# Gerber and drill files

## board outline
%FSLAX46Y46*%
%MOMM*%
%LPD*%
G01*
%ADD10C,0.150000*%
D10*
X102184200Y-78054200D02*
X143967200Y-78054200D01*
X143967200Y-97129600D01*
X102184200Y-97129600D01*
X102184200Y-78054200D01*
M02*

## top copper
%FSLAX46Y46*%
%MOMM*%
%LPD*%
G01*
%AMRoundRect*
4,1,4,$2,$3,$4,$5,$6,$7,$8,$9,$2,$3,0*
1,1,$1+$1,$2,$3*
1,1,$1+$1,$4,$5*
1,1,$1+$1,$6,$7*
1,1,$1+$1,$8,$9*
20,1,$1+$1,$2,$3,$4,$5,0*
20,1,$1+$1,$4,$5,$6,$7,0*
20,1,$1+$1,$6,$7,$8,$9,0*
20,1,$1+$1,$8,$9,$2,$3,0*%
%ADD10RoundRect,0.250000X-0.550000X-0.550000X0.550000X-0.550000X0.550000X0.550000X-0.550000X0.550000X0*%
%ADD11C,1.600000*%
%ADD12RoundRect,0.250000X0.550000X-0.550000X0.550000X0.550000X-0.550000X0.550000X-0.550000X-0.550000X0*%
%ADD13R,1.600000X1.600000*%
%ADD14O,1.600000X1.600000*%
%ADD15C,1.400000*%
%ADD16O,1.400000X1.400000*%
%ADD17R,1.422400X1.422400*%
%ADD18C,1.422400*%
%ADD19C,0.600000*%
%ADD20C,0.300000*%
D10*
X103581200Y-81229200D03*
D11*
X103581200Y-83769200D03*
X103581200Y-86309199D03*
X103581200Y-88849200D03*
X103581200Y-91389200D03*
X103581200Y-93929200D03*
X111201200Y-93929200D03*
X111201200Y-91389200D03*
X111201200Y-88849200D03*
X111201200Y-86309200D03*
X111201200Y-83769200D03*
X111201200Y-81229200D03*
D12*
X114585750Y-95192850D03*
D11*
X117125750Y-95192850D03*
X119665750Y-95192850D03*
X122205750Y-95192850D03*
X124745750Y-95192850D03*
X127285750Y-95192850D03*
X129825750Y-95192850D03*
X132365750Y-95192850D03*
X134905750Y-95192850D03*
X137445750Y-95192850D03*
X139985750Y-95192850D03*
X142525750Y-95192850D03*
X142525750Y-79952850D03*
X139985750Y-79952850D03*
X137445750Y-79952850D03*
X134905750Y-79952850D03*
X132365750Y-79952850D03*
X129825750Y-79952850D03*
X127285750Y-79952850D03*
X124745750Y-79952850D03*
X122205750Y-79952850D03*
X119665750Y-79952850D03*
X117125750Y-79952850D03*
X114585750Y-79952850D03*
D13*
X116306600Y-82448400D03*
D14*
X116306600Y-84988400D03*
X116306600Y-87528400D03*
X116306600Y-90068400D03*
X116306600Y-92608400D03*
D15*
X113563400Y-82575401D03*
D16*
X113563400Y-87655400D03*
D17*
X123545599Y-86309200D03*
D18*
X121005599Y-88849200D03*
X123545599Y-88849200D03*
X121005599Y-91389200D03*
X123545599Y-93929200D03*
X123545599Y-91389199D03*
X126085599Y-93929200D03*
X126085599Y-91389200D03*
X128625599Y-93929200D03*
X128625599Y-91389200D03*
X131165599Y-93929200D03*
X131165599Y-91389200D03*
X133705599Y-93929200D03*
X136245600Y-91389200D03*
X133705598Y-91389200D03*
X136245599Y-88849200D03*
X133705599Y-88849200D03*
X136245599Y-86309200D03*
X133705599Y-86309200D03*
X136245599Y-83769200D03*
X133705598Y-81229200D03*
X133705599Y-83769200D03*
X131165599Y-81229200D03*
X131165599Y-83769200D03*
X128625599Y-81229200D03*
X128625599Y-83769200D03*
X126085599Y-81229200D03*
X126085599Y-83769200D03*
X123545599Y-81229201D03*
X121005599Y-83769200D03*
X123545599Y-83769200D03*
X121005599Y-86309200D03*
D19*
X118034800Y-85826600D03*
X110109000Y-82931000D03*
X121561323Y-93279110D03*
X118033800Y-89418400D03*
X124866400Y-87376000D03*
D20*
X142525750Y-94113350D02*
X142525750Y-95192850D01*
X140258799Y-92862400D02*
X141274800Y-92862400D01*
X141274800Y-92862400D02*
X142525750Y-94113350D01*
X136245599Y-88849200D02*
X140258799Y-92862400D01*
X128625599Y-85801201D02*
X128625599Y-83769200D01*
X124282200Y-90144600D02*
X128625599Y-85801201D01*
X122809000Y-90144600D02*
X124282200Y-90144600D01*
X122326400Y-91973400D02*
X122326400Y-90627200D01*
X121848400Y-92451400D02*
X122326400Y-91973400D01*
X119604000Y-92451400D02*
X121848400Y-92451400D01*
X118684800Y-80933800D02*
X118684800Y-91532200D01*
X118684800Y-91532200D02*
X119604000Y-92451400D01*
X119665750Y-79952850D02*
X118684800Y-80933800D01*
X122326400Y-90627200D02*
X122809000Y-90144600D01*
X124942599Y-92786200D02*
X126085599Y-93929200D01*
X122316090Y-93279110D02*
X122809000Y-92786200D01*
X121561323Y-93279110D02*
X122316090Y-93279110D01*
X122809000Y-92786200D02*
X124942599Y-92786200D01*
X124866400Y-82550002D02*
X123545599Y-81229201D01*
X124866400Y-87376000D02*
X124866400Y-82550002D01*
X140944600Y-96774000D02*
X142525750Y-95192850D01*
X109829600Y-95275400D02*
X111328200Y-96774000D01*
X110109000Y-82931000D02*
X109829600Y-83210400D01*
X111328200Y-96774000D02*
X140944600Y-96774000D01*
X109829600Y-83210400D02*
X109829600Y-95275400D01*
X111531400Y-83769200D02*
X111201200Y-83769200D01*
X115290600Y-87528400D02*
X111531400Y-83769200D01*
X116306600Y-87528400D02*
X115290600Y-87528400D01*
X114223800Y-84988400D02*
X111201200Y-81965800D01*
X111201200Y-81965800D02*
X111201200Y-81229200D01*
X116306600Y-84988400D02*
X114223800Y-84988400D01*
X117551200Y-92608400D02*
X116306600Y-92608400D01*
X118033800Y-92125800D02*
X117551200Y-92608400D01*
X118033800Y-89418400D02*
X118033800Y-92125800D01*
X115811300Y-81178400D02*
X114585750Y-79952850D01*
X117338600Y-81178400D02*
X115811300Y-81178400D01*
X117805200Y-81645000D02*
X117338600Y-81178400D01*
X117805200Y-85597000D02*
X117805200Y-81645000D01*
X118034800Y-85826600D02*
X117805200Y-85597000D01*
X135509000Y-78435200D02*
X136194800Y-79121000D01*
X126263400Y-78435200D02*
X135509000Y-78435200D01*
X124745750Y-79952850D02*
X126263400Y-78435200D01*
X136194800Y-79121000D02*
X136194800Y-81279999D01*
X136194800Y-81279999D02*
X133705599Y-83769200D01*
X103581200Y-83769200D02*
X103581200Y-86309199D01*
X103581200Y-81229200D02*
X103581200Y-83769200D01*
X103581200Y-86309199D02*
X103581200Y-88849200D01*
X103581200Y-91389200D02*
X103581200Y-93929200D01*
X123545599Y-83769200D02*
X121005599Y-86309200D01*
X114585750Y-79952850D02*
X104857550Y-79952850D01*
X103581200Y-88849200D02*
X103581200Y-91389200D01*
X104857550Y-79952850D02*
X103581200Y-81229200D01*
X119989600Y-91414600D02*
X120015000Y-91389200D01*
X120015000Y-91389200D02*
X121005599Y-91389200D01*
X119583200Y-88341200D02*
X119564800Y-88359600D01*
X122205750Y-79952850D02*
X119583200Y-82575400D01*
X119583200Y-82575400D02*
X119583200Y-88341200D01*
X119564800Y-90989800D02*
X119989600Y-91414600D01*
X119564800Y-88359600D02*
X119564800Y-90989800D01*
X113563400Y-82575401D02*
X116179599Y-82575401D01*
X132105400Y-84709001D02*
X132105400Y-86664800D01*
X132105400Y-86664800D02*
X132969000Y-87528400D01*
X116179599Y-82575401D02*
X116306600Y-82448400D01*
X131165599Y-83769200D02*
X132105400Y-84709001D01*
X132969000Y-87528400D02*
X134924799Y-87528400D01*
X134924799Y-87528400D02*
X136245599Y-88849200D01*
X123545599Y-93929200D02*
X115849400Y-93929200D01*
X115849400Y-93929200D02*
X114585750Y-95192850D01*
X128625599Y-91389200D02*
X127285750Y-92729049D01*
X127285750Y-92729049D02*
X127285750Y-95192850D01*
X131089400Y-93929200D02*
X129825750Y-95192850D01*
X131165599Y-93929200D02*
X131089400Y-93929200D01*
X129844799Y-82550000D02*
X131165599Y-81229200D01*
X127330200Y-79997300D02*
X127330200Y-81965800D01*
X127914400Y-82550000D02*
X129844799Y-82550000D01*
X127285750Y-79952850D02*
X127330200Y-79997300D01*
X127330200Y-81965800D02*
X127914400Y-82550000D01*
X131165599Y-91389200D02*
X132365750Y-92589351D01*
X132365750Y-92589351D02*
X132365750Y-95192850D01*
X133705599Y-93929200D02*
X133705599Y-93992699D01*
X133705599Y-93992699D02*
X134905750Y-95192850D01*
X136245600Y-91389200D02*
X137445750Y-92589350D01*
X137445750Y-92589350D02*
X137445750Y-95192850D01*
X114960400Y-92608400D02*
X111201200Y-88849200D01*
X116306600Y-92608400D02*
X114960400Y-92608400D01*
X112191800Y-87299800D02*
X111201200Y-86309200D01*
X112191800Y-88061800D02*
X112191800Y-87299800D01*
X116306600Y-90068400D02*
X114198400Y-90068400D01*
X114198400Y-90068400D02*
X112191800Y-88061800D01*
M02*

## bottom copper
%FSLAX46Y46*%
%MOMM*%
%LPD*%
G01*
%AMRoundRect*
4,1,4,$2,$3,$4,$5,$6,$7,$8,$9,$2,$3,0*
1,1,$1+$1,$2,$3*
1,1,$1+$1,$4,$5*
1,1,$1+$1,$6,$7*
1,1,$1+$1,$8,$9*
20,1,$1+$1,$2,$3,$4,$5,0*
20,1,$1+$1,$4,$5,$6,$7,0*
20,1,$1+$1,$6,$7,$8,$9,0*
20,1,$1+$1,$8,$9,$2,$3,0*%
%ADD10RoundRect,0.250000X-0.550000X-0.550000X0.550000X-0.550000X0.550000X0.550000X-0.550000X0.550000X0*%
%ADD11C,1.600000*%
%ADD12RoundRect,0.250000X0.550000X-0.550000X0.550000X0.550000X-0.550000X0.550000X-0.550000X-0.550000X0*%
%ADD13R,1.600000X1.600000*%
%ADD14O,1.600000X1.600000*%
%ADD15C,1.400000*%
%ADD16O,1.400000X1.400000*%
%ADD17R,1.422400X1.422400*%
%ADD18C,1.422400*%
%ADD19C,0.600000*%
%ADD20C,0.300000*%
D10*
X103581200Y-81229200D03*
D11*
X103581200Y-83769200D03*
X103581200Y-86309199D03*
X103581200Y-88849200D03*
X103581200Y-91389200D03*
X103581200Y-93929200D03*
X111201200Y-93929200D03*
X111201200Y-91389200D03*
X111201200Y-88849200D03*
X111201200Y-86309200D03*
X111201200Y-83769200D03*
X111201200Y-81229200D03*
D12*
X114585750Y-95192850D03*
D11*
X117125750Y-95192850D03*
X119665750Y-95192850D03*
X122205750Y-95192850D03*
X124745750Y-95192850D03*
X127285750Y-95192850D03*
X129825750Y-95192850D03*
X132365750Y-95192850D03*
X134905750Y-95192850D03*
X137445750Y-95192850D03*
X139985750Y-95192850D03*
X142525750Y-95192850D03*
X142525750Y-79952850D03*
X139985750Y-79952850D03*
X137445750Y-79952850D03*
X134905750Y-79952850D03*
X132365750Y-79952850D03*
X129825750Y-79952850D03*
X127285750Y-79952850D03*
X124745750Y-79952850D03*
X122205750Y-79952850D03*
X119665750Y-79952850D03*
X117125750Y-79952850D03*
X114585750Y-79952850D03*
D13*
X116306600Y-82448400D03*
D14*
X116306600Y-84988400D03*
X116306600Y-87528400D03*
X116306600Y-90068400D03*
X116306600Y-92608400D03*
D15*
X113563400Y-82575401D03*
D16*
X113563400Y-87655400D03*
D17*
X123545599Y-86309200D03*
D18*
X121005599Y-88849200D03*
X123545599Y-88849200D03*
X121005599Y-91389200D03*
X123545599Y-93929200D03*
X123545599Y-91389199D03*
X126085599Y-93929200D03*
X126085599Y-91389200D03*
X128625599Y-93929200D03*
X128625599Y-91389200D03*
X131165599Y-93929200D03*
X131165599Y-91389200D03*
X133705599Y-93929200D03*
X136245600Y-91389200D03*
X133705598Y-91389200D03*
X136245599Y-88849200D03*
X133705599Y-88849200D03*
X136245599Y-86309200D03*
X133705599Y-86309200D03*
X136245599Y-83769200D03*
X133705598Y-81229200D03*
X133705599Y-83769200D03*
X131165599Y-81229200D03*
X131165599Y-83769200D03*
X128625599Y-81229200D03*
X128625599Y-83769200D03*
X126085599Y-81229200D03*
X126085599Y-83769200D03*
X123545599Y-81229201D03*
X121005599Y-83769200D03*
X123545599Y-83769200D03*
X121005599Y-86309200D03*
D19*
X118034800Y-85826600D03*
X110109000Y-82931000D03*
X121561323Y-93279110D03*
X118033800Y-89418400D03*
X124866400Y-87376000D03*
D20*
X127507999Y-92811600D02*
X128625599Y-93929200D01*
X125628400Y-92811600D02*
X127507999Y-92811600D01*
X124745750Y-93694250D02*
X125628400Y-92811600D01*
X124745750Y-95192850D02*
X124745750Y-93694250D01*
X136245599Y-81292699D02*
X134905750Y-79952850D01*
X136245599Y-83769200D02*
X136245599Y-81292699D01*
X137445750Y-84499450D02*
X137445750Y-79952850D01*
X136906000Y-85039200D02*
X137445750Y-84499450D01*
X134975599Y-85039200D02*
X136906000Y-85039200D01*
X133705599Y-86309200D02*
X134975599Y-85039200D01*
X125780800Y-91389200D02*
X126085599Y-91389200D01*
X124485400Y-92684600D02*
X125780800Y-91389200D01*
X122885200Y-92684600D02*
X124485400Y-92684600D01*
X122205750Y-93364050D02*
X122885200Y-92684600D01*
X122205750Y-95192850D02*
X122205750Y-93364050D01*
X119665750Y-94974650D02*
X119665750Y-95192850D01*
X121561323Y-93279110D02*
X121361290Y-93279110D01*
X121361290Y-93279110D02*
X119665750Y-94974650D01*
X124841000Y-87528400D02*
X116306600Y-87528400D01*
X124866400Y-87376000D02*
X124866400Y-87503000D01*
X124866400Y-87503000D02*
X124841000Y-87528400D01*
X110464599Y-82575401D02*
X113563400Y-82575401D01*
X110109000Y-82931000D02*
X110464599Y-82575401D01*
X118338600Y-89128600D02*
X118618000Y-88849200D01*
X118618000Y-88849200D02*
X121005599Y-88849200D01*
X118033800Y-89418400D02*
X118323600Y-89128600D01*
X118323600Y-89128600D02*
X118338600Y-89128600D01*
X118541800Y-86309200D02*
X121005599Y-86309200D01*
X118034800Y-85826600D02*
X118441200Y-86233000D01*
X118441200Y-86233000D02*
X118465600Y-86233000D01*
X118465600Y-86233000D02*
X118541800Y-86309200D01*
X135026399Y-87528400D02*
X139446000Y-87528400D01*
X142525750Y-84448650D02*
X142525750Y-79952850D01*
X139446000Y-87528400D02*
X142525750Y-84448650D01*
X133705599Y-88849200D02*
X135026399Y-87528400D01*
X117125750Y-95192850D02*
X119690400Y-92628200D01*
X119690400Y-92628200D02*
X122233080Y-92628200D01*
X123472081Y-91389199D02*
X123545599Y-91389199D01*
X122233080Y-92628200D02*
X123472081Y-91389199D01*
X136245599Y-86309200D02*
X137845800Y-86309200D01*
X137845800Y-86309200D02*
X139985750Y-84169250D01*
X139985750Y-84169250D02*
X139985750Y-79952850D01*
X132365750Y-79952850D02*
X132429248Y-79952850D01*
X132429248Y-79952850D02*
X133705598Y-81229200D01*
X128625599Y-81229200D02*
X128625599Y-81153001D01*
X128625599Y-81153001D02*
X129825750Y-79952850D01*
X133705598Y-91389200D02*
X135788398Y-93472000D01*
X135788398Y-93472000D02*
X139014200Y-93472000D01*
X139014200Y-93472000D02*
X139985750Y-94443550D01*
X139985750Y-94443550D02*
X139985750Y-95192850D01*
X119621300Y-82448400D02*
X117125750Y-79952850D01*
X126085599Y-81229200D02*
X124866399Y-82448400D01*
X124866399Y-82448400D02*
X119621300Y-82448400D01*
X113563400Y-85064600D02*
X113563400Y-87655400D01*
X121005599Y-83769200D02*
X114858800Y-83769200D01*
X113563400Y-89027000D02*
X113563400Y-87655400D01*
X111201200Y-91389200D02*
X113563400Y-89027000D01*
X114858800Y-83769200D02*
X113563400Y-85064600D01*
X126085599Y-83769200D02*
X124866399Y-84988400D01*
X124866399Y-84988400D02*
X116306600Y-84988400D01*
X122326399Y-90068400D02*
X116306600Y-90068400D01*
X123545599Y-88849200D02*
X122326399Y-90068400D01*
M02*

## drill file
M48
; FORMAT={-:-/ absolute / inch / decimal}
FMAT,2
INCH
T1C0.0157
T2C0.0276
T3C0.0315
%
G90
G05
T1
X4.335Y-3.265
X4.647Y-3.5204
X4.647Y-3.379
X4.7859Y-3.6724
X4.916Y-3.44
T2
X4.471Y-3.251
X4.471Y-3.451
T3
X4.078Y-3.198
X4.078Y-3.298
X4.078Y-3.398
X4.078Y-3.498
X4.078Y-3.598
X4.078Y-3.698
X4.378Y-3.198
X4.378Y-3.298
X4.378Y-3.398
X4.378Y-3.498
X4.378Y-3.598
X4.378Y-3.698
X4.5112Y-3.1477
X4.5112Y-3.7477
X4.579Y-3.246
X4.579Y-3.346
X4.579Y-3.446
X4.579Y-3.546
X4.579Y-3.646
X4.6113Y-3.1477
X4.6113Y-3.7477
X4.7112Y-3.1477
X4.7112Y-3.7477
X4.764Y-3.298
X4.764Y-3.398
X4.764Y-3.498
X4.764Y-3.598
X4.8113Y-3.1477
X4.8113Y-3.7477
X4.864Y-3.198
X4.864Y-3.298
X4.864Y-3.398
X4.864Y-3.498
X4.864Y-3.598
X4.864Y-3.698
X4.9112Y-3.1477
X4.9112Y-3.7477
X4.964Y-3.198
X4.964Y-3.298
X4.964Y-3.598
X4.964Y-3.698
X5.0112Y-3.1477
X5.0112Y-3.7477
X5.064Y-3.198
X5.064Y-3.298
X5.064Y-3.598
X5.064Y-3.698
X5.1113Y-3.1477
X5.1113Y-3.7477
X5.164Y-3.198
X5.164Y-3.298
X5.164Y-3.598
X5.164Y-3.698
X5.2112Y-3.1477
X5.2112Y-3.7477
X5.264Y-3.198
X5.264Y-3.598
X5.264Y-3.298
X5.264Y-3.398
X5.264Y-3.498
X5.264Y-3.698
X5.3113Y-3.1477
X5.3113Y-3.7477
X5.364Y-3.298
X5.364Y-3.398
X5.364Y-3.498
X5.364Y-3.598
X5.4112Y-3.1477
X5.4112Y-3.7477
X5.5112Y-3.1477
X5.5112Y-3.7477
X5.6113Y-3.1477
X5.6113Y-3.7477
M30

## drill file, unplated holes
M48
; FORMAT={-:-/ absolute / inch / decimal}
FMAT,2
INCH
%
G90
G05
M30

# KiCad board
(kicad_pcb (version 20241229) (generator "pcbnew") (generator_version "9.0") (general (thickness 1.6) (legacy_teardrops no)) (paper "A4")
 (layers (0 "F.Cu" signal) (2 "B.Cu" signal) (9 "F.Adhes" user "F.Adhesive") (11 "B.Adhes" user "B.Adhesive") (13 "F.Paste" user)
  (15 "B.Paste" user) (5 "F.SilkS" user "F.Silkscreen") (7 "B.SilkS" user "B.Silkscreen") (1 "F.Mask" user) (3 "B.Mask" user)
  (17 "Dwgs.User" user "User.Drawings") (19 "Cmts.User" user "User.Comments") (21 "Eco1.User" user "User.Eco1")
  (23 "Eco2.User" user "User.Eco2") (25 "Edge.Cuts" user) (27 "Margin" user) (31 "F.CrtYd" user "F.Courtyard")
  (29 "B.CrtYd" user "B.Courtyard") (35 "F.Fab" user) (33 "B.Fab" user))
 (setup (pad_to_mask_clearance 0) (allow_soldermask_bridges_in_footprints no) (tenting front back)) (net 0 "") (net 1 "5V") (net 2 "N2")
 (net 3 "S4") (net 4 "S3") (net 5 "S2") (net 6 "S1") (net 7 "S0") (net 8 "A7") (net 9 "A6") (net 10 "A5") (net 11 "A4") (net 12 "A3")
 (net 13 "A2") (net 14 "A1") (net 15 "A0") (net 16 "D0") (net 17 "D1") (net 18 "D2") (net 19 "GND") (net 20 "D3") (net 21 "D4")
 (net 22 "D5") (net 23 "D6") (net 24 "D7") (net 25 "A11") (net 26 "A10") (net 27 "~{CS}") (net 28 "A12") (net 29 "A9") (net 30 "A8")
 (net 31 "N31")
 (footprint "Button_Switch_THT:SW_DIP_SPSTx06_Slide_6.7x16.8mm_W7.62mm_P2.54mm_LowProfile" (layer "F.Cu") (at 103.5812 81.2292)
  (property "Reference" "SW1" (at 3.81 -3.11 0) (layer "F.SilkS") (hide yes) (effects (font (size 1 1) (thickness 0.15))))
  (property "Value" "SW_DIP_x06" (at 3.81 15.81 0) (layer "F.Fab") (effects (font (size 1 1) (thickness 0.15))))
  (pad "1" thru_hole roundrect (at 0 0) (size 1.6 1.6) (drill 0.8) (layers "*.Cu" "*.Mask") (remove_unused_layers no)
   (roundrect_rratio 0.15625) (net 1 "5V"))
  (pad "2" thru_hole circle (at 0 2.54) (size 1.6 1.6) (drill 0.8) (layers "*.Cu" "*.Mask") (remove_unused_layers no) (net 1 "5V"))
  (pad "3" thru_hole circle (at 0 5.079999) (size 1.6 1.6) (drill 0.8) (layers "*.Cu" "*.Mask") (remove_unused_layers no) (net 1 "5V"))
  (pad "4" thru_hole circle (at 0 7.62) (size 1.6 1.6) (drill 0.8) (layers "*.Cu" "*.Mask") (remove_unused_layers no) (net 1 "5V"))
  (pad "5" thru_hole circle (at 0 10.16) (size 1.6 1.6) (drill 0.8) (layers "*.Cu" "*.Mask") (remove_unused_layers no) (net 1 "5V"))
  (pad "6" thru_hole circle (at 0 12.7) (size 1.6 1.6) (drill 0.8) (layers "*.Cu" "*.Mask") (remove_unused_layers no) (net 1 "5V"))
  (pad "7" thru_hole circle (at 7.62 12.7) (size 1.6 1.6) (drill 0.8) (layers "*.Cu" "*.Mask") (remove_unused_layers no) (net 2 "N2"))
  (pad "8" thru_hole circle (at 7.62 10.16) (size 1.6 1.6) (drill 0.8) (layers "*.Cu" "*.Mask") (remove_unused_layers no) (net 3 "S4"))
  (pad "9" thru_hole circle (at 7.62 7.62) (size 1.6 1.6) (drill 0.8) (layers "*.Cu" "*.Mask") (remove_unused_layers no) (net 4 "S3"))
  (pad "10" thru_hole circle (at 7.62 5.08) (size 1.6 1.6) (drill 0.8) (layers "*.Cu" "*.Mask") (remove_unused_layers no) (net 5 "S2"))
  (pad "11" thru_hole circle (at 7.62 2.54) (size 1.6 1.6) (drill 0.8) (layers "*.Cu" "*.Mask") (remove_unused_layers no) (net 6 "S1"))
  (pad "12" thru_hole circle (at 7.62 0) (size 1.6 1.6) (drill 0.8) (layers "*.Cu" "*.Mask") (remove_unused_layers no) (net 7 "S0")))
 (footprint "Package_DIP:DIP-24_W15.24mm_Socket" (layer "F.Cu") (at 114.58575 95.19285 90)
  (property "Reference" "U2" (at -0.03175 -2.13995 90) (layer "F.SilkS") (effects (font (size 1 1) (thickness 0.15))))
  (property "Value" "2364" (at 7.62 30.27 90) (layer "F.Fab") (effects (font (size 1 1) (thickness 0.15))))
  (pad "1" thru_hole roundrect (at 0 0 90) (size 1.6 1.6) (drill 0.8) (layers "*.Cu" "*.Mask") (remove_unused_layers no)
   (roundrect_rratio 0.15625) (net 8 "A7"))
  (pad "2" thru_hole circle (at 0 2.54 90) (size 1.6 1.6) (drill 0.8) (layers "*.Cu" "*.Mask") (remove_unused_layers no) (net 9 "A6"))
  (pad "3" thru_hole circle (at 0 5.08 90) (size 1.6 1.6) (drill 0.8) (layers "*.Cu" "*.Mask") (remove_unused_layers no) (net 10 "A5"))
  (pad "4" thru_hole circle (at 0 7.62 90) (size 1.6 1.6) (drill 0.8) (layers "*.Cu" "*.Mask") (remove_unused_layers no) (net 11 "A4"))
  (pad "5" thru_hole circle (at 0 10.16 90) (size 1.6 1.6) (drill 0.8) (layers "*.Cu" "*.Mask") (remove_unused_layers no) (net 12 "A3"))
  (pad "6" thru_hole circle (at 0 12.7 90) (size 1.6 1.6) (drill 0.8) (layers "*.Cu" "*.Mask") (remove_unused_layers no) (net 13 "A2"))
  (pad "7" thru_hole circle (at 0 15.24 90) (size 1.6 1.6) (drill 0.8) (layers "*.Cu" "*.Mask") (remove_unused_layers no) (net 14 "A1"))
  (pad "8" thru_hole circle (at 0 17.78 90) (size 1.6 1.6) (drill 0.8) (layers "*.Cu" "*.Mask") (remove_unused_layers no) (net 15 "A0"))
  (pad "9" thru_hole circle (at 0 20.32 90) (size 1.6 1.6) (drill 0.8) (layers "*.Cu" "*.Mask") (remove_unused_layers no) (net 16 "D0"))
  (pad "10" thru_hole circle (at 0 22.86 90) (size 1.6 1.6) (drill 0.8) (layers "*.Cu" "*.Mask") (remove_unused_layers no) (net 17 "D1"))
  (pad "11" thru_hole circle (at 0 25.4 90) (size 1.6 1.6) (drill 0.8) (layers "*.Cu" "*.Mask") (remove_unused_layers no) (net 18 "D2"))
  (pad "12" thru_hole circle (at 0 27.94 90) (size 1.6 1.6) (drill 0.8) (layers "*.Cu" "*.Mask") (remove_unused_layers no) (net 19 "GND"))
  (pad "13" thru_hole circle (at 15.24 27.94 90) (size 1.6 1.6) (drill 0.8) (layers "*.Cu" "*.Mask") (remove_unused_layers no) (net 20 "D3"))
  (pad "14" thru_hole circle (at 15.24 25.4 90) (size 1.6 1.6) (drill 0.8) (layers "*.Cu" "*.Mask") (remove_unused_layers no) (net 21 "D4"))
  (pad "15" thru_hole circle (at 15.24 22.86 90) (size 1.6 1.6) (drill 0.8) (layers "*.Cu" "*.Mask") (remove_unused_layers no) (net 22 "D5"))
  (pad "16" thru_hole circle (at 15.24 20.32 90) (size 1.6 1.6) (drill 0.8) (layers "*.Cu" "*.Mask") (remove_unused_layers no) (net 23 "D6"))
  (pad "17" thru_hole circle (at 15.24 17.78 90) (size 1.6 1.6) (drill 0.8) (layers "*.Cu" "*.Mask") (remove_unused_layers no) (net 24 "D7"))
  (pad "18" thru_hole circle (at 15.24 15.24 90) (size 1.6 1.6) (drill 0.8) (layers "*.Cu" "*.Mask") (remove_unused_layers no)
   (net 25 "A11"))
  (pad "19" thru_hole circle (at 15.24 12.7 90) (size 1.6 1.6) (drill 0.8) (layers "*.Cu" "*.Mask") (remove_unused_layers no) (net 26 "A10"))
  (pad "20" thru_hole circle (at 15.24 10.16 90) (size 1.6 1.6) (drill 0.8) (layers "*.Cu" "*.Mask") (remove_unused_layers no)
   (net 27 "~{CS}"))
  (pad "21" thru_hole circle (at 15.24 7.62 90) (size 1.6 1.6) (drill 0.8) (layers "*.Cu" "*.Mask") (remove_unused_layers no) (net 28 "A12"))
  (pad "22" thru_hole circle (at 15.24 5.08 90) (size 1.6 1.6) (drill 0.8) (layers "*.Cu" "*.Mask") (remove_unused_layers no) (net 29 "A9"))
  (pad "23" thru_hole circle (at 15.24 2.54 90) (size 1.6 1.6) (drill 0.8) (layers "*.Cu" "*.Mask") (remove_unused_layers no) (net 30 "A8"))
  (pad "24" thru_hole circle (at 15.24 0 90) (size 1.6 1.6) (drill 0.8) (layers "*.Cu" "*.Mask") (remove_unused_layers no) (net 1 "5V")))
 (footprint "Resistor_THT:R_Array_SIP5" (layer "F.Cu") (at 116.3066 82.4484 -90)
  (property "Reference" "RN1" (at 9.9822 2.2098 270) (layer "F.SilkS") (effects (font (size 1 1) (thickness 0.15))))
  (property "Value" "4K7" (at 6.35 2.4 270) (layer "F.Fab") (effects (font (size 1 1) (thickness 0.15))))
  (pad "1" thru_hole rect (at 0 0 270) (size 1.6 1.6) (drill 0.8) (layers "*.Cu" "*.Mask") (remove_unused_layers no) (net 19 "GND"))
  (pad "2" thru_hole oval (at 2.54 0 270) (size 1.6 1.6) (drill 0.8) (layers "*.Cu" "*.Mask") (remove_unused_layers no) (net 7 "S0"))
  (pad "3" thru_hole oval (at 5.08 0 270) (size 1.6 1.6) (drill 0.8) (layers "*.Cu" "*.Mask") (remove_unused_layers no) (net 6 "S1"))
  (pad "4" thru_hole oval (at 7.62 0 270) (size 1.6 1.6) (drill 0.8) (layers "*.Cu" "*.Mask") (remove_unused_layers no) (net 5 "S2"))
  (pad "5" thru_hole oval (at 10.16 0 270) (size 1.6 1.6) (drill 0.8) (layers "*.Cu" "*.Mask") (remove_unused_layers no) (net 4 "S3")))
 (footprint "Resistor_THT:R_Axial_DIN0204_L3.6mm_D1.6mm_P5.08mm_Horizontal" (layer "F.Cu") (at 113.5634 82.575401 -90)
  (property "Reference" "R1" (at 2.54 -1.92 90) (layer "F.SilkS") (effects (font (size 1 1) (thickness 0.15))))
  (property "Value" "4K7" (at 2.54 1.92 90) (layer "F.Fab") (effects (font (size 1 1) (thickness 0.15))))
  (pad "1" thru_hole circle (at 0 0 270) (size 1.4 1.4) (drill 0.7) (layers "*.Cu" "*.Mask") (remove_unused_layers no) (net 19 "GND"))
  (pad "2" thru_hole oval (at 5.079999 0 270) (size 1.4 1.4) (drill 0.7) (layers "*.Cu" "*.Mask") (remove_unused_layers no) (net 3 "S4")))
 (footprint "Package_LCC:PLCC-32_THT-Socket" (layer "F.Cu") (at 123.545599 86.3092 90)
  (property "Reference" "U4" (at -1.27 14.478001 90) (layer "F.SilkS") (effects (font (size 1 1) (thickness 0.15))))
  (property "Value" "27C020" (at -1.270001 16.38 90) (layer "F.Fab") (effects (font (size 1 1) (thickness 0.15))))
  (pad "1" thru_hole rect (at 0 0 90) (size 1.4224 1.4224) (drill 0.8) (layers "*.Cu" "*.Mask") (remove_unused_layers no) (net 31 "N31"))
  (pad "2" thru_hole circle (at -2.54 -2.54 90) (size 1.4224 1.4224) (drill 0.8) (layers "*.Cu" "*.Mask") (remove_unused_layers no)
   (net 4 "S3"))
  (pad "3" thru_hole circle (at -2.54 0 90) (size 1.4224 1.4224) (drill 0.8) (layers "*.Cu" "*.Mask") (remove_unused_layers no) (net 5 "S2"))
  (pad "4" thru_hole circle (at -5.08 -2.54 90) (size 1.4224 1.4224) (drill 0.8) (layers "*.Cu" "*.Mask") (remove_unused_layers no)
   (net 28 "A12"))
  (pad "5" thru_hole circle (at -7.62 0 90) (size 1.4224 1.4224) (drill 0.8) (layers "*.Cu" "*.Mask") (remove_unused_layers no) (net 8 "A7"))
  (pad "6" thru_hole circle (at -5.079999 0 90) (size 1.4224 1.4224) (drill 0.8) (layers "*.Cu" "*.Mask") (remove_unused_layers no)
   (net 9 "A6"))
  (pad "7" thru_hole circle (at -7.62 2.54 90) (size 1.4224 1.4224) (drill 0.8) (layers "*.Cu" "*.Mask") (remove_unused_layers no)
   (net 10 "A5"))
  (pad "8" thru_hole circle (at -5.08 2.54 90) (size 1.4224 1.4224) (drill 0.8) (layers "*.Cu" "*.Mask") (remove_unused_layers no)
   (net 11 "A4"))
  (pad "9" thru_hole circle (at -7.62 5.08 90) (size 1.4224 1.4224) (drill 0.8) (layers "*.Cu" "*.Mask") (remove_unused_layers no)
   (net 12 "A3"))
  (pad "10" thru_hole circle (at -5.08 5.08 90) (size 1.4224 1.4224) (drill 0.8) (layers "*.Cu" "*.Mask") (remove_unused_layers no)
   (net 13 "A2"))
  (pad "11" thru_hole circle (at -7.62 7.62 90) (size 1.4224 1.4224) (drill 0.8) (layers "*.Cu" "*.Mask") (remove_unused_layers no)
   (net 14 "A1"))
  (pad "12" thru_hole circle (at -5.08 7.62 90) (size 1.4224 1.4224) (drill 0.8) (layers "*.Cu" "*.Mask") (remove_unused_layers no)
   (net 15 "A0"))
  (pad "13" thru_hole circle (at -7.62 10.16 90) (size 1.4224 1.4224) (drill 0.8) (layers "*.Cu" "*.Mask") (remove_unused_layers no)
   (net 16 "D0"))
  (pad "14" thru_hole circle (at -5.08 12.700001 90) (size 1.4224 1.4224) (drill 0.8) (layers "*.Cu" "*.Mask") (remove_unused_layers no)
   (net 17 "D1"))
  (pad "15" thru_hole circle (at -5.08 10.159999 90) (size 1.4224 1.4224) (drill 0.8) (layers "*.Cu" "*.Mask") (remove_unused_layers no)
   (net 18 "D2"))
  (pad "16" thru_hole circle (at -2.54 12.7 90) (size 1.4224 1.4224) (drill 0.8) (layers "*.Cu" "*.Mask") (remove_unused_layers no)
   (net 19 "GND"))
  (pad "17" thru_hole circle (at -2.54 10.16 90) (size 1.4224 1.4224) (drill 0.8) (layers "*.Cu" "*.Mask") (remove_unused_layers no)
   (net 20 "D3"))
  (pad "18" thru_hole circle (at 0 12.7 90) (size 1.4224 1.4224) (drill 0.8) (layers "*.Cu" "*.Mask") (remove_unused_layers no)
   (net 21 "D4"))
  (pad "19" thru_hole circle (at 0 10.16 90) (size 1.4224 1.4224) (drill 0.8) (layers "*.Cu" "*.Mask") (remove_unused_layers no)
   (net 22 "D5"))
  (pad "20" thru_hole circle (at 2.54 12.7 90) (size 1.4224 1.4224) (drill 0.8) (layers "*.Cu" "*.Mask") (remove_unused_layers no)
   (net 23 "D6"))
  (pad "21" thru_hole circle (at 5.08 10.159999 90) (size 1.4224 1.4224) (drill 0.8) (layers "*.Cu" "*.Mask") (remove_unused_layers no)
   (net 24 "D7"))
  (pad "22" thru_hole circle (at 2.54 10.16 90) (size 1.4224 1.4224) (drill 0.8) (layers "*.Cu" "*.Mask") (remove_unused_layers no)
   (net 27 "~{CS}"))
  (pad "23" thru_hole circle (at 5.08 7.62 90) (size 1.4224 1.4224) (drill 0.8) (layers "*.Cu" "*.Mask") (remove_unused_layers no)
   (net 26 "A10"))
  (pad "24" thru_hole circle (at 2.54 7.62 90) (size 1.4224 1.4224) (drill 0.8) (layers "*.Cu" "*.Mask") (remove_unused_layers no)
   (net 19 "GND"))
  (pad "25" thru_hole circle (at 5.08 5.08 90) (size 1.4224 1.4224) (drill 0.8) (layers "*.Cu" "*.Mask") (remove_unused_layers no)
   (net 25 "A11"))
  (pad "26" thru_hole circle (at 2.54 5.08 90) (size 1.4224 1.4224) (drill 0.8) (layers "*.Cu" "*.Mask") (remove_unused_layers no)
   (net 29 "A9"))
  (pad "27" thru_hole circle (at 5.08 2.54 90) (size 1.4224 1.4224) (drill 0.8) (layers "*.Cu" "*.Mask") (remove_unused_layers no)
   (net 30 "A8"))
  (pad "28" thru_hole circle (at 2.54 2.54 90) (size 1.4224 1.4224) (drill 0.8) (layers "*.Cu" "*.Mask") (remove_unused_layers no)
   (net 7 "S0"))
  (pad "29" thru_hole circle (at 5.079999 0 90) (size 1.4224 1.4224) (drill 0.8) (layers "*.Cu" "*.Mask") (remove_unused_layers no)
   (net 6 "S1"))
  (pad "30" thru_hole circle (at 2.54 -2.54 90) (size 1.4224 1.4224) (drill 0.8) (layers "*.Cu" "*.Mask") (remove_unused_layers no)
   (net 3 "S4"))
  (pad "31" thru_hole circle (at 2.54 0 90) (size 1.4224 1.4224) (drill 0.8) (layers "*.Cu" "*.Mask") (remove_unused_layers no) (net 1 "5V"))
  (pad "32" thru_hole circle (at 0 -2.54 90) (size 1.4224 1.4224) (drill 0.8) (layers "*.Cu" "*.Mask") (remove_unused_layers no)
   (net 1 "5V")))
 (gr_rect (start 102.1842 78.0542) (end 143.9672 97.1296) (stroke (width 0.15) (type default)) (fill no) (layer "Edge.Cuts"))
 (segment (start 135.509 78.4352) (end 136.1948 79.121) (width 0.3) (layer "F.Cu") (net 27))
 (segment (start 126.2634 78.4352) (end 135.509 78.4352) (width 0.3) (layer "F.Cu") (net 27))
 (segment (start 124.74575 79.95285) (end 126.2634 78.4352) (width 0.3) (layer "F.Cu") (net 27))
 (segment (start 136.1948 79.121) (end 136.1948 81.279999) (width 0.3) (layer "F.Cu") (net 27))
 (segment (start 136.1948 81.279999) (end 133.705599 83.7692) (width 0.3) (layer "F.Cu") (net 27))
 (segment (start 117.8052 85.597) (end 117.8052 81.645) (width 0.3) (layer "F.Cu") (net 1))
 (segment (start 103.5812 83.7692) (end 103.5812 86.309199) (width 0.3) (layer "F.Cu") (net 1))
 (segment (start 103.5812 81.2292) (end 103.5812 83.7692) (width 0.3) (layer "F.Cu") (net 1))
 (segment (start 103.5812 86.309199) (end 103.5812 88.8492) (width 0.3) (layer "F.Cu") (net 1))
 (segment (start 103.5812 91.3892) (end 103.5812 93.9292) (width 0.3) (layer "F.Cu") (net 1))
 (segment (start 123.545599 83.7692) (end 121.005599 86.3092) (width 0.3) (layer "F.Cu") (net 1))
 (segment (start 117.8052 81.645) (end 117.3386 81.1784) (width 0.3) (layer "F.Cu") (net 1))
 (segment (start 114.58575 79.95285) (end 104.85755 79.95285) (width 0.3) (layer "F.Cu") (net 1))
 (segment (start 103.5812 88.8492) (end 103.5812 91.3892) (width 0.3) (layer "F.Cu") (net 1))
 (segment (start 117.3386 81.1784) (end 115.8113 81.1784) (width 0.3) (layer "F.Cu") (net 1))
 (segment (start 104.85755 79.95285) (end 103.5812 81.2292) (width 0.3) (layer "F.Cu") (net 1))
 (segment (start 115.8113 81.1784) (end 114.58575 79.95285) (width 0.3) (layer "F.Cu") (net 1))
 (segment (start 118.0348 85.8266) (end 117.8052 85.597) (width 0.3) (layer "F.Cu") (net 1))
 (via (at 118.0348 85.8266) (size 0.6) (drill 0.4) (layers "F.Cu" "B.Cu") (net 1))
 (segment (start 118.5418 86.3092) (end 121.005599 86.3092) (width 0.3) (layer "B.Cu") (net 1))
 (segment (start 118.4656 86.233) (end 118.5418 86.3092) (width 0.3) (layer "B.Cu") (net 1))
 (segment (start 118.0348 85.8266) (end 118.4412 86.233) (width 0.3) (layer "B.Cu") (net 1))
 (segment (start 118.4412 86.233) (end 118.4656 86.233) (width 0.3) (layer "B.Cu") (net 1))
 (segment (start 119.9896 91.4146) (end 120.015 91.3892) (width 0.3) (layer "F.Cu") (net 28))
 (segment (start 120.015 91.3892) (end 121.005599 91.3892) (width 0.3) (layer "F.Cu") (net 28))
 (segment (start 119.5832 88.3412) (end 119.5648 88.3596) (width 0.3) (layer "F.Cu") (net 28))
 (segment (start 122.20575 79.95285) (end 119.5832 82.5754) (width 0.3) (layer "F.Cu") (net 28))
 (segment (start 119.5832 82.5754) (end 119.5832 88.3412) (width 0.3) (layer "F.Cu") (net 28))
 (segment (start 119.5648 90.9898) (end 119.9896 91.4146) (width 0.3) (layer "F.Cu") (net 28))
 (segment (start 119.5648 88.3596) (end 119.5648 90.9898) (width 0.3) (layer "F.Cu") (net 28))
 (segment (start 136.245599 88.8492) (end 140.258799 92.8624) (width 0.3) (layer "F.Cu") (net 19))
 (segment (start 113.5634 82.575401) (end 116.179599 82.575401) (width 0.3) (layer "F.Cu") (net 19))
 (segment (start 132.1054 84.709001) (end 132.1054 86.6648) (width 0.3) (layer "F.Cu") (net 19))
 (segment (start 132.1054 86.6648) (end 132.969 87.5284) (width 0.3) (layer "F.Cu") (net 19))
 (segment (start 111.3282 96.774) (end 140.9446 96.774) (width 0.3) (layer "F.Cu") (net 19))
 (segment (start 141.2748 92.8624) (end 142.52575 94.11335) (width 0.3) (layer "F.Cu") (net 19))
 (segment (start 142.52575 94.11335) (end 142.52575 95.19285) (width 0.3) (layer "F.Cu") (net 19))
 (segment (start 140.9446 96.774) (end 142.52575 95.19285) (width 0.3) (layer "F.Cu") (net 19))
 (segment (start 110.109 82.931) (end 109.8296 83.2104) (width 0.3) (layer "F.Cu") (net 19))
 (segment (start 109.8296 83.2104) (end 109.8296 95.2754) (width 0.3) (layer "F.Cu") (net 19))
 (segment (start 109.8296 95.2754) (end 111.3282 96.774) (width 0.3) (layer "F.Cu") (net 19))
 (segment (start 116.179599 82.575401) (end 116.3066 82.4484) (width 0.3) (layer "F.Cu") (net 19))
 (segment (start 131.165599 83.7692) (end 132.1054 84.709001) (width 0.3) (layer "F.Cu") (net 19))
 (segment (start 132.969 87.5284) (end 134.924799 87.5284) (width 0.3) (layer "F.Cu") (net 19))
 (segment (start 140.258799 92.8624) (end 141.2748 92.8624) (width 0.3) (layer "F.Cu") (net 19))
 (segment (start 134.924799 87.5284) (end 136.245599 88.8492) (width 0.3) (layer "F.Cu") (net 19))
 (via (at 110.109 82.931) (size 0.6) (drill 0.4) (layers "F.Cu" "B.Cu") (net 19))
 (segment (start 110.464599 82.575401) (end 113.5634 82.575401) (width 0.3) (layer "B.Cu") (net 19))
 (segment (start 110.109 82.931) (end 110.464599 82.575401) (width 0.3) (layer "B.Cu") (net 19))
 (segment (start 123.545599 93.9292) (end 115.8494 93.9292) (width 0.3) (layer "F.Cu") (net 8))
 (segment (start 115.8494 93.9292) (end 114.58575 95.19285) (width 0.3) (layer "F.Cu") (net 8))
 (segment (start 135.026399 87.5284) (end 139.446 87.5284) (width 0.3) (layer "B.Cu") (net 20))
 (segment (start 142.52575 84.44865) (end 142.52575 79.95285) (width 0.3) (layer "B.Cu") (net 20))
 (segment (start 139.446 87.5284) (end 142.52575 84.44865) (width 0.3) (layer "B.Cu") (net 20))
 (segment (start 133.705599 88.8492) (end 135.026399 87.5284) (width 0.3) (layer "B.Cu") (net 20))
 (segment (start 117.12575 95.19285) (end 119.6904 92.6282) (width 0.3) (layer "B.Cu") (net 9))
 (segment (start 119.6904 92.6282) (end 122.23308 92.6282) (width 0.3) (layer "B.Cu") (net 9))
 (segment (start 123.472081 91.389199) (end 123.545599 91.389199) (width 0.3) (layer "B.Cu") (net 9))
 (segment (start 122.23308 92.6282) (end 123.472081 91.389199) (width 0.3) (layer "B.Cu") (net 9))
 (segment (start 136.245599 86.3092) (end 137.8458 86.3092) (width 0.3) (layer "B.Cu") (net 21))
 (segment (start 137.8458 86.3092) (end 139.98575 84.16925) (width 0.3) (layer "B.Cu") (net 21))
 (segment (start 139.98575 84.16925) (end 139.98575 79.95285) (width 0.3) (layer "B.Cu") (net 21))
 (segment (start 122.31609 93.27911) (end 122.809 92.7862) (width 0.3) (layer "F.Cu") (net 10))
 (segment (start 124.942599 92.7862) (end 126.085599 93.9292) (width 0.3) (layer "F.Cu") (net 10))
 (segment (start 121.561323 93.27911) (end 122.31609 93.27911) (width 0.3) (layer "F.Cu") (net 10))
 (segment (start 122.809 92.7862) (end 124.942599 92.7862) (width 0.3) (layer "F.Cu") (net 10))
 (via (at 121.561323 93.27911) (size 0.6) (drill 0.4) (layers "F.Cu" "B.Cu") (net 10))
 (segment (start 119.66575 94.97465) (end 119.66575 95.19285) (width 0.3) (layer "B.Cu") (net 10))
 (segment (start 121.561323 93.27911) (end 121.36129 93.27911) (width 0.3) (layer "B.Cu") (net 10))
 (segment (start 121.36129 93.27911) (end 119.66575 94.97465) (width 0.3) (layer "B.Cu") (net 10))
 (segment (start 133.705599 86.3092) (end 134.975599 85.0392) (width 0.3) (layer "B.Cu") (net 22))
 (segment (start 136.906 85.0392) (end 137.44575 84.49945) (width 0.3) (layer "B.Cu") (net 22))
 (segment (start 137.44575 84.49945) (end 137.44575 79.95285) (width 0.3) (layer "B.Cu") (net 22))
 (segment (start 134.975599 85.0392) (end 136.906 85.0392) (width 0.3) (layer "B.Cu") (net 22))
 (segment (start 125.7808 91.3892) (end 126.085599 91.3892) (width 0.3) (layer "B.Cu") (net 11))
 (segment (start 122.8852 92.6846) (end 124.4854 92.6846) (width 0.3) (layer "B.Cu") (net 11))
 (segment (start 122.20575 93.36405) (end 122.8852 92.6846) (width 0.3) (layer "B.Cu") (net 11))
 (segment (start 122.20575 95.19285) (end 122.20575 93.36405) (width 0.3) (layer "B.Cu") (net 11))
 (segment (start 124.4854 92.6846) (end 125.7808 91.3892) (width 0.3) (layer "B.Cu") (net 11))
 (segment (start 136.245599 81.292699) (end 134.90575 79.95285) (width 0.3) (layer "B.Cu") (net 23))
 (segment (start 136.245599 83.7692) (end 136.245599 81.292699) (width 0.3) (layer "B.Cu") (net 23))
 (segment (start 125.6284 92.8116) (end 127.507999 92.8116) (width 0.3) (layer "B.Cu") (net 12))
 (segment (start 124.74575 93.69425) (end 125.6284 92.8116) (width 0.3) (layer "B.Cu") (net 12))
 (segment (start 124.74575 95.19285) (end 124.74575 93.69425) (width 0.3) (layer "B.Cu") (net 12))
 (segment (start 127.507999 92.8116) (end 128.625599 93.9292) (width 0.3) (layer "B.Cu") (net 12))
 (segment (start 132.36575 79.95285) (end 132.429248 79.95285) (width 0.3) (layer "B.Cu") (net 24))
 (segment (start 132.429248 79.95285) (end 133.705598 81.2292) (width 0.3) (layer "B.Cu") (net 24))
 (segment (start 128.625599 91.3892) (end 127.28575 92.729049) (width 0.3) (layer "F.Cu") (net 13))
 (segment (start 127.28575 92.729049) (end 127.28575 95.19285) (width 0.3) (layer "F.Cu") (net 13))
 (segment (start 128.625599 81.2292) (end 128.625599 81.153001) (width 0.3) (layer "B.Cu") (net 25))
 (segment (start 128.625599 81.153001) (end 129.82575 79.95285) (width 0.3) (layer "B.Cu") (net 25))
 (segment (start 131.0894 93.9292) (end 129.82575 95.19285) (width 0.3) (layer "F.Cu") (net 14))
 (segment (start 131.165599 93.9292) (end 131.0894 93.9292) (width 0.3) (layer "F.Cu") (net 14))
 (segment (start 129.844799 82.55) (end 131.165599 81.2292) (width 0.3) (layer "F.Cu") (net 26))
 (segment (start 127.3302 79.9973) (end 127.3302 81.9658) (width 0.3) (layer "F.Cu") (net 26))
 (segment (start 127.9144 82.55) (end 129.844799 82.55) (width 0.3) (layer "F.Cu") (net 26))
 (segment (start 127.28575 79.95285) (end 127.3302 79.9973) (width 0.3) (layer "F.Cu") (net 26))
 (segment (start 127.3302 81.9658) (end 127.9144 82.55) (width 0.3) (layer "F.Cu") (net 26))
 (segment (start 131.165599 91.3892) (end 132.36575 92.589351) (width 0.3) (layer "F.Cu") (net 15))
 (segment (start 132.36575 92.589351) (end 132.36575 95.19285) (width 0.3) (layer "F.Cu") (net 15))
 (segment (start 133.705599 93.9292) (end 133.705599 93.992699) (width 0.3) (layer "F.Cu") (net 16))
 (segment (start 133.705599 93.992699) (end 134.90575 95.19285) (width 0.3) (layer "F.Cu") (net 16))
 (segment (start 136.2456 91.3892) (end 137.44575 92.58935) (width 0.3) (layer "F.Cu") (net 17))
 (segment (start 137.44575 92.58935) (end 137.44575 95.19285) (width 0.3) (layer "F.Cu") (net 17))
 (segment (start 122.3264 91.9734) (end 122.3264 90.6272) (width 0.3) (layer "F.Cu") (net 29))
 (segment (start 118.6848 80.9338) (end 118.6848 91.5322) (width 0.3) (layer "F.Cu") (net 29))
 (segment (start 121.8484 92.4514) (end 122.3264 91.9734) (width 0.3) (layer "F.Cu") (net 29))
 (segment (start 118.6848 91.5322) (end 119.604 92.4514) (width 0.3) (layer "F.Cu") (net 29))
 (segment (start 124.2822 90.1446) (end 128.625599 85.801201) (width 0.3) (layer "F.Cu") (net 29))
 (segment (start 128.625599 85.801201) (end 128.625599 83.7692) (width 0.3) (layer "F.Cu") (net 29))
 (segment (start 122.3264 90.6272) (end 122.809 90.1446) (width 0.3) (layer "F.Cu") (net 29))
 (segment (start 119.66575 79.95285) (end 118.6848 80.9338) (width 0.3) (layer "F.Cu") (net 29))
 (segment (start 122.809 90.1446) (end 124.2822 90.1446) (width 0.3) (layer "F.Cu") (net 29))
 (segment (start 119.604 92.4514) (end 121.8484 92.4514) (width 0.3) (layer "F.Cu") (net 29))
 (segment (start 133.705598 91.3892) (end 135.788398 93.472) (width 0.3) (layer "B.Cu") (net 18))
 (segment (start 135.788398 93.472) (end 139.0142 93.472) (width 0.3) (layer "B.Cu") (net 18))
 (segment (start 139.0142 93.472) (end 139.98575 94.44355) (width 0.3) (layer "B.Cu") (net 18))
 (segment (start 139.98575 94.44355) (end 139.98575 95.19285) (width 0.3) (layer "B.Cu") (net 18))
 (segment (start 119.6213 82.4484) (end 117.12575 79.95285) (width 0.3) (layer "B.Cu") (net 30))
 (segment (start 126.085599 81.2292) (end 124.866399 82.4484) (width 0.3) (layer "B.Cu") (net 30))
 (segment (start 124.866399 82.4484) (end 119.6213 82.4484) (width 0.3) (layer "B.Cu") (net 30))
 (segment (start 113.5634 85.0646) (end 113.5634 87.6554) (width 0.3) (layer "B.Cu") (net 3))
 (segment (start 121.005599 83.7692) (end 114.8588 83.7692) (width 0.3) (layer "B.Cu") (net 3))
 (segment (start 113.5634 89.027) (end 113.5634 87.6554) (width 0.3) (layer "B.Cu") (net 3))
 (segment (start 111.2012 91.3892) (end 113.5634 89.027) (width 0.3) (layer "B.Cu") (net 3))
 (segment (start 114.8588 83.7692) (end 113.5634 85.0646) (width 0.3) (layer "B.Cu") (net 3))
 (segment (start 114.2238 84.9884) (end 111.2012 81.9658) (width 0.3) (layer "F.Cu") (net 7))
 (segment (start 111.2012 81.9658) (end 111.2012 81.2292) (width 0.3) (layer "F.Cu") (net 7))
 (segment (start 116.3066 84.9884) (end 114.2238 84.9884) (width 0.3) (layer "F.Cu") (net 7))
 (segment (start 126.085599 83.7692) (end 124.866399 84.9884) (width 0.3) (layer "B.Cu") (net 7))
 (segment (start 124.866399 84.9884) (end 116.3066 84.9884) (width 0.3) (layer "B.Cu") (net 7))
 (segment (start 118.0338 92.1258) (end 117.5512 92.6084) (width 0.3) (layer "F.Cu") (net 4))
 (segment (start 118.0338 89.4184) (end 118.0338 92.1258) (width 0.3) (layer "F.Cu") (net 4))
 (segment (start 114.9604 92.6084) (end 111.2012 88.8492) (width 0.3) (layer "F.Cu") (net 4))
 (segment (start 116.3066 92.6084) (end 114.9604 92.6084) (width 0.3) (layer "F.Cu") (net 4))
 (segment (start 117.5512 92.6084) (end 116.3066 92.6084) (width 0.3) (layer "F.Cu") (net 4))
 (via (at 118.0338 89.4184) (size 0.6) (drill 0.4) (layers "F.Cu" "B.Cu") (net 4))
 (segment (start 118.0338 89.4184) (end 118.3236 89.1286) (width 0.3) (layer "B.Cu") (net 4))
 (segment (start 118.618 88.8492) (end 121.005599 88.8492) (width 0.3) (layer "B.Cu") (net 4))
 (segment (start 118.3236 89.1286) (end 118.3386 89.1286) (width 0.3) (layer "B.Cu") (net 4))
 (segment (start 118.3386 89.1286) (end 118.618 88.8492) (width 0.3) (layer "B.Cu") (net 4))
 (segment (start 112.1918 87.2998) (end 111.2012 86.3092) (width 0.3) (layer "F.Cu") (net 5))
 (segment (start 112.1918 88.0618) (end 112.1918 87.2998) (width 0.3) (layer "F.Cu") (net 5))
 (segment (start 116.3066 90.0684) (end 114.1984 90.0684) (width 0.3) (layer "F.Cu") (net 5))
 (segment (start 114.1984 90.0684) (end 112.1918 88.0618) (width 0.3) (layer "F.Cu") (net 5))
 (segment (start 122.326399 90.0684) (end 116.3066 90.0684) (width 0.3) (layer "B.Cu") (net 5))
 (segment (start 123.545599 88.8492) (end 122.326399 90.0684) (width 0.3) (layer "B.Cu") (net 5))
 (segment (start 124.8664 82.550002) (end 123.545599 81.229201) (width 0.3) (layer "F.Cu") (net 6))
 (segment (start 115.2906 87.5284) (end 111.5314 83.7692) (width 0.3) (layer "F.Cu") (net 6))
 (segment (start 111.5314 83.7692) (end 111.2012 83.7692) (width 0.3) (layer "F.Cu") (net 6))
 (segment (start 124.8664 87.376) (end 124.8664 82.550002) (width 0.3) (layer "F.Cu") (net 6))
 (segment (start 116.3066 87.5284) (end 115.2906 87.5284) (width 0.3) (layer "F.Cu") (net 6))
 (via (at 124.8664 87.376) (size 0.6) (drill 0.4) (layers "F.Cu" "B.Cu") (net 6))
 (segment (start 124.8664 87.376) (end 124.8664 87.503) (width 0.3) (layer "B.Cu") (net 6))
 (segment (start 124.8664 87.503) (end 124.841 87.5284) (width 0.3) (layer "B.Cu") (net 6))
 (segment (start 124.841 87.5284) (end 116.3066 87.5284) (width 0.3) (layer "B.Cu") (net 6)))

